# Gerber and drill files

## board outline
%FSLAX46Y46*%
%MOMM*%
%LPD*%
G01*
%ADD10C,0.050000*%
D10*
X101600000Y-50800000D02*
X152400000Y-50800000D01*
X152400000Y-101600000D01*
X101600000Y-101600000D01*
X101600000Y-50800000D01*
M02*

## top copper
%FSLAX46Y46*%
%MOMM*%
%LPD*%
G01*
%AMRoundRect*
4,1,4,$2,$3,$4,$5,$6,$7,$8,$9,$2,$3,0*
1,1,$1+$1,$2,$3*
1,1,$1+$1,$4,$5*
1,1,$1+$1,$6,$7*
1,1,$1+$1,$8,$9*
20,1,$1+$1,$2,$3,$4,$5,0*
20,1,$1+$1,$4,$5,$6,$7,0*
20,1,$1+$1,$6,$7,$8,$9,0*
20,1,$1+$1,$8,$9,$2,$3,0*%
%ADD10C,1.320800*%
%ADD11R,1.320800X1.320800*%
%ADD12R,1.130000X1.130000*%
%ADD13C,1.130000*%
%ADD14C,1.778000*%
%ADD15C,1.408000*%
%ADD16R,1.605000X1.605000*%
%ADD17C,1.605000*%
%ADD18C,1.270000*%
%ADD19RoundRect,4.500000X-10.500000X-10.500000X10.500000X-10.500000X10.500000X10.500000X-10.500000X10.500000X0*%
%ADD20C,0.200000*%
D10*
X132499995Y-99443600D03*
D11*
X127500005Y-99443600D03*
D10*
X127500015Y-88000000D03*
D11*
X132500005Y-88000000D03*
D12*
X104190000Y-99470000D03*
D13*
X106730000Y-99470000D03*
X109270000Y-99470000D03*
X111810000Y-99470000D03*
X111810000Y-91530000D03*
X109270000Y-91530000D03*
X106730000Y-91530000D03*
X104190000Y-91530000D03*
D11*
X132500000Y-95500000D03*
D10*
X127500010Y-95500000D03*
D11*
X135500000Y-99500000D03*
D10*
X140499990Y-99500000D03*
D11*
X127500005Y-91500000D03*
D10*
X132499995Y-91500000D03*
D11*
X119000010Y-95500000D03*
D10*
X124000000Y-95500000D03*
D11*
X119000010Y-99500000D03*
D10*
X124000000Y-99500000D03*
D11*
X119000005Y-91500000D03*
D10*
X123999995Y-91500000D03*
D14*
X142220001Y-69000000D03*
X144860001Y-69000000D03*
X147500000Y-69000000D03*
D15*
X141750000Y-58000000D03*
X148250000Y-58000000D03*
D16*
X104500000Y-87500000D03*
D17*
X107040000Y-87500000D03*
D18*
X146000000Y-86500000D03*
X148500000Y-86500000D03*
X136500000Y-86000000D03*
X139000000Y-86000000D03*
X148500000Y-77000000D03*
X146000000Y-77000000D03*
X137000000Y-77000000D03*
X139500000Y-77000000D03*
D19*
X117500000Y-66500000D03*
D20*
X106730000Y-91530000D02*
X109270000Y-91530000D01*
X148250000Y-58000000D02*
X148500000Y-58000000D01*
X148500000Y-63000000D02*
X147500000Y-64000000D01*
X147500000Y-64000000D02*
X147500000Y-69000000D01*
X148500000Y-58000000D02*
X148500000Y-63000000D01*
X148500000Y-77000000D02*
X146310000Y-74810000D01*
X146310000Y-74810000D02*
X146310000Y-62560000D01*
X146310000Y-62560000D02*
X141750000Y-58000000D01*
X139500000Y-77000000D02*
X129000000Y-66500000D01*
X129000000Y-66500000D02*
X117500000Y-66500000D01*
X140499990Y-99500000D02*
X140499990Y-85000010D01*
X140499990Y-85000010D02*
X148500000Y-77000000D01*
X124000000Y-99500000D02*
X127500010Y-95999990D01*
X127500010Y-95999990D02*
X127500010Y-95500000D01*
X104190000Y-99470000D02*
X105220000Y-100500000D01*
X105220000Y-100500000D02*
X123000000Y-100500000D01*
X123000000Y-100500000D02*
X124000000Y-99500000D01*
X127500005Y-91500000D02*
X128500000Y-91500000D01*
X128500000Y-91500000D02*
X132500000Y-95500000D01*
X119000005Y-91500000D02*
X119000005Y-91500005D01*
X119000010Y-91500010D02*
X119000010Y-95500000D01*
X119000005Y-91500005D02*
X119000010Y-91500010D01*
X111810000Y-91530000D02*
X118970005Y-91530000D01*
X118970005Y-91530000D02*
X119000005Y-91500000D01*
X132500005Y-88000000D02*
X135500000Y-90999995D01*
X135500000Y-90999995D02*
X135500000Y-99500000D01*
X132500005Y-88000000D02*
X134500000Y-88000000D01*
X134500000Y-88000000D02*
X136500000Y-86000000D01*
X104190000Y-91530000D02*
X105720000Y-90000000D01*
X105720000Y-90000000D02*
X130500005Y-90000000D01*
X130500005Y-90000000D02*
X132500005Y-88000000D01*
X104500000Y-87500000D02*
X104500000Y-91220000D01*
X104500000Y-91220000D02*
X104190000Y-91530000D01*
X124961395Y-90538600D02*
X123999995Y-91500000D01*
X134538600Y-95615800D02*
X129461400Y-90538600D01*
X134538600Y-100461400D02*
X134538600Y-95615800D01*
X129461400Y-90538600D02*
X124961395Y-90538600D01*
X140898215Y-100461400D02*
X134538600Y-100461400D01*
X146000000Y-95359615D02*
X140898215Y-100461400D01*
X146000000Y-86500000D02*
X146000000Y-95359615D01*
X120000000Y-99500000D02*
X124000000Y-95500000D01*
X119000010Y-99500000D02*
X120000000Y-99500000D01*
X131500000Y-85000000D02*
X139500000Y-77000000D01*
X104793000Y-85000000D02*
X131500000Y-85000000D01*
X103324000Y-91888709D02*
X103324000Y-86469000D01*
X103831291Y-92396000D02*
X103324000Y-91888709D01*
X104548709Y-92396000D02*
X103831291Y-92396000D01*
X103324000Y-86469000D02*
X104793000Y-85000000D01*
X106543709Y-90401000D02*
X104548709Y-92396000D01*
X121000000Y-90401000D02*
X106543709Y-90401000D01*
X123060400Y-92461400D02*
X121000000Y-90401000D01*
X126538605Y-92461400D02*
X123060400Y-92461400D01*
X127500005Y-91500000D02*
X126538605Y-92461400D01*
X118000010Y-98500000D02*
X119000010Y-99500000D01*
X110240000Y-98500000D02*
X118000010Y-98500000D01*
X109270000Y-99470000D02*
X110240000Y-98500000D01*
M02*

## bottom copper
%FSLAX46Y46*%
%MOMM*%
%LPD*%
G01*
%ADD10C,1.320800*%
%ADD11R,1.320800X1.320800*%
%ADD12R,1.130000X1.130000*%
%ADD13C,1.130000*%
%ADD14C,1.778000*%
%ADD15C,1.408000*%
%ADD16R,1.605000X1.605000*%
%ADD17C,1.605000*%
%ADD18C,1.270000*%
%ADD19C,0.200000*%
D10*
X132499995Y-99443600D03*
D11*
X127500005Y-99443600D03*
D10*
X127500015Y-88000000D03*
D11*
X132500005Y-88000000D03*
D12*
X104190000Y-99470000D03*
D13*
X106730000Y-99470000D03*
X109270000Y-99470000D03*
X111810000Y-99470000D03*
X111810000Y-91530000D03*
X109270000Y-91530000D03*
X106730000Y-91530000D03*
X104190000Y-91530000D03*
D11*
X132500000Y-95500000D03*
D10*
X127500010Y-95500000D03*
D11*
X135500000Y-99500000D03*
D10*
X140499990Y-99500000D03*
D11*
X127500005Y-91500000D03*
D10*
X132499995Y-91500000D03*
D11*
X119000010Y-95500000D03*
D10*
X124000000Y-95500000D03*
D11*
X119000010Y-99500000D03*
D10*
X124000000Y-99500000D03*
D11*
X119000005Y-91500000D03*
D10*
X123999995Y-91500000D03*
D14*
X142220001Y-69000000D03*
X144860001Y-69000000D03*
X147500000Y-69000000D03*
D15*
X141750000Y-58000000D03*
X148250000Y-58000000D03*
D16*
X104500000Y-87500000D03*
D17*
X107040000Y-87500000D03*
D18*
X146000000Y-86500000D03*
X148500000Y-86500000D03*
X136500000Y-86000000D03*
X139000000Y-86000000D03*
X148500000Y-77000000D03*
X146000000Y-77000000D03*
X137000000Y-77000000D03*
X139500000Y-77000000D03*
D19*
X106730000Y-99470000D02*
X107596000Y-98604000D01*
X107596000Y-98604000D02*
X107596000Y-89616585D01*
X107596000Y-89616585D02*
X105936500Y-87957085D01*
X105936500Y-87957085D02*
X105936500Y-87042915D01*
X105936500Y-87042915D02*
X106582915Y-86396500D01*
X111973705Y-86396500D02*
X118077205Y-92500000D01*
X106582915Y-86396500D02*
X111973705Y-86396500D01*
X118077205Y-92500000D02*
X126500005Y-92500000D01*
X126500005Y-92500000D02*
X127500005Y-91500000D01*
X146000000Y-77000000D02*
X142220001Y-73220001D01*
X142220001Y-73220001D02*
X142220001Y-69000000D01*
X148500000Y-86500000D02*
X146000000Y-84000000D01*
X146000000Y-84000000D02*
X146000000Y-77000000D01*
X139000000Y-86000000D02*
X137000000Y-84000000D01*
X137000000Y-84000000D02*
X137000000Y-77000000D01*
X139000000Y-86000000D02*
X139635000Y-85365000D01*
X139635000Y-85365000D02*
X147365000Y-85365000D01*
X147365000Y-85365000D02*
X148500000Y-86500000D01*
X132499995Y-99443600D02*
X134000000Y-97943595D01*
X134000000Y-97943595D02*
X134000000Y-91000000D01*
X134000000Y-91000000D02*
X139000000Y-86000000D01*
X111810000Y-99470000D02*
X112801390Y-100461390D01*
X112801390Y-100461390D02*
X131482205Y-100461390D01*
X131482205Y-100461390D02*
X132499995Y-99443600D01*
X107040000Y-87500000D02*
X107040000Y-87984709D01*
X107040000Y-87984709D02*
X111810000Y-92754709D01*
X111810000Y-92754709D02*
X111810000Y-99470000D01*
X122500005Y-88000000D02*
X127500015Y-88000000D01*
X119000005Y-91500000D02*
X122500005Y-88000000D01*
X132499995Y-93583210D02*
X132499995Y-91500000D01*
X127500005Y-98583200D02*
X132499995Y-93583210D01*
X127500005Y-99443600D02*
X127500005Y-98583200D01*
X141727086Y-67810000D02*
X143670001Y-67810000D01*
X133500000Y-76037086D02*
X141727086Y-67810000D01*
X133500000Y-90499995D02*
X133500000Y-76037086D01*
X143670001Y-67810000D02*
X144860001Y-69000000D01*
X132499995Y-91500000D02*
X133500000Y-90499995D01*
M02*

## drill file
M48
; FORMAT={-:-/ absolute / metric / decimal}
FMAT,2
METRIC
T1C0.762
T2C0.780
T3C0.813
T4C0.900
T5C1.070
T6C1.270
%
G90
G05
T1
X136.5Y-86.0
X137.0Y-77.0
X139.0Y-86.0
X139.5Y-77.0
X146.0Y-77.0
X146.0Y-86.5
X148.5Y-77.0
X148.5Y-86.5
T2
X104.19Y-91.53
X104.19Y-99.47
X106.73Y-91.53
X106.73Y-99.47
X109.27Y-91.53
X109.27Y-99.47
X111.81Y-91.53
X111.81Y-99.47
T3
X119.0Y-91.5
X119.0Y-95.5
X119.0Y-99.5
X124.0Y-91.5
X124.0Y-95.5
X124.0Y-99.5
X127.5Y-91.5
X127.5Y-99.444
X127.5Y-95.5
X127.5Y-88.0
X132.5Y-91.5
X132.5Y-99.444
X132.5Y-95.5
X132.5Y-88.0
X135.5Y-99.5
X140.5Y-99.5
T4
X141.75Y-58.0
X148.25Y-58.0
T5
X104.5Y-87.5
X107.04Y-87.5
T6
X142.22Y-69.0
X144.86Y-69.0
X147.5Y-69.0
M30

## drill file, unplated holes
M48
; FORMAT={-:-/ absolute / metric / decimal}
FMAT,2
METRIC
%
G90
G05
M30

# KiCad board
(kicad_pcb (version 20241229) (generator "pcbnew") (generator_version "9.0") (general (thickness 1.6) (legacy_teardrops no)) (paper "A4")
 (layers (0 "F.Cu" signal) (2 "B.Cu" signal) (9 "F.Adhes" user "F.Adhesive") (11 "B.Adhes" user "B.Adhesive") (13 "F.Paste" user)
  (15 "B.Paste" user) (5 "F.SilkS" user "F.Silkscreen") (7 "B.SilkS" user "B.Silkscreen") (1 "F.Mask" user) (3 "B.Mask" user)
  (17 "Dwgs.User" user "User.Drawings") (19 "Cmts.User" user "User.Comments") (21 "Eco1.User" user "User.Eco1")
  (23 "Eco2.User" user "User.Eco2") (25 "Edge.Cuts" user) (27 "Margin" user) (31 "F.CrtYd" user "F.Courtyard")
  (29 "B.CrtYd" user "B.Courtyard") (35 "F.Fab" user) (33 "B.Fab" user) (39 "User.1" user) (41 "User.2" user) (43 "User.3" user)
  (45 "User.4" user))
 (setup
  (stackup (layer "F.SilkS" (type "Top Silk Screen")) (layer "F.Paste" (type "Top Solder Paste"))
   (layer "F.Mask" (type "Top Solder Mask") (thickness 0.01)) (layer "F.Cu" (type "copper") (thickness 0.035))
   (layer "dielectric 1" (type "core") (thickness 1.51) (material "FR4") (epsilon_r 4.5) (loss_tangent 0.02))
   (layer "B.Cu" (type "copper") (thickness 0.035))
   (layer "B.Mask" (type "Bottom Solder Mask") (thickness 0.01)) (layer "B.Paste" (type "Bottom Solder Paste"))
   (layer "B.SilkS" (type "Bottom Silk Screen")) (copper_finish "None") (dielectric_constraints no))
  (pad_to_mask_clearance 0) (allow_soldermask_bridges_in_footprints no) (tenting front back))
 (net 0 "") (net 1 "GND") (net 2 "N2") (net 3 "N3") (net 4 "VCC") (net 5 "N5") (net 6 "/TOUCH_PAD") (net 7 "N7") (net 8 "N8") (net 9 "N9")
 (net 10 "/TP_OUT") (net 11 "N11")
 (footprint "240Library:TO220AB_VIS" (layer "F.Cu") (at 142.220001 69)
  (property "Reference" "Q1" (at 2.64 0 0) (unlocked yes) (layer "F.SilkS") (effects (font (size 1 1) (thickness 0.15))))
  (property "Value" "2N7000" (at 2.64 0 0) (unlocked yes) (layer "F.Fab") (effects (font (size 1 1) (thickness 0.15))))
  (pad "1" thru_hole circle (at 0 0) (size 1.778 1.778) (drill 1.27) (layers "*.Cu" "*.Mask") (remove_unused_layers no) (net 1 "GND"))
  (pad "2" thru_hole circle (at 2.64 0) (size 1.778 1.778) (drill 1.27) (layers "*.Cu" "*.Mask") (remove_unused_layers no) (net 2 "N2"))
  (pad "3" thru_hole circle (at 5.279999 0) (size 1.778 1.778) (drill 1.27) (layers "*.Cu" "*.Mask") (remove_unused_layers no) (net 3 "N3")))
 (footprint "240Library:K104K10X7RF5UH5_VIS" (layer "F.Cu") (at 132.500005 88 180)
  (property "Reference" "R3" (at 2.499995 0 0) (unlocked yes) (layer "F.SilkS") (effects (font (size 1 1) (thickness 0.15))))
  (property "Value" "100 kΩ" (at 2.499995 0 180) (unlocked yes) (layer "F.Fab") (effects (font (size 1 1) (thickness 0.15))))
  (pad "1" thru_hole rect (at 0 0 180) (size 1.3208 1.3208) (drill 0.8128) (layers "*.Cu" "*.Mask") (remove_unused_layers no) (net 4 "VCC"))
  (pad "2" thru_hole circle (at 4.99999 0 180) (size 1.3208 1.3208) (drill 0.8128) (layers "*.Cu" "*.Mask") (remove_unused_layers no)
   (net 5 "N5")))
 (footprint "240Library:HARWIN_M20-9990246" (layer "F.Cu") (at 105.77 87.5)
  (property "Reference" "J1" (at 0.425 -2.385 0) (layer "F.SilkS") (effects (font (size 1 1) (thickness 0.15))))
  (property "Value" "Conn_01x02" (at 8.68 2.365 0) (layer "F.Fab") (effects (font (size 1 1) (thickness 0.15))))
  (pad "1" thru_hole rect (at -1.27 0) (size 1.605 1.605) (drill 1.07) (layers "*.Cu" "*.Mask") (remove_unused_layers no) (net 4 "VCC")
   (solder_mask_margin 0.102))
  (pad "2" thru_hole circle (at 1.27 0) (size 1.605 1.605) (drill 1.07) (layers "*.Cu" "*.Mask") (remove_unused_layers no) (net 1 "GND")
   (solder_mask_margin 0.102)))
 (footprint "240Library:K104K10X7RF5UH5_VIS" (layer "F.Cu") (at 127.500005 91.5)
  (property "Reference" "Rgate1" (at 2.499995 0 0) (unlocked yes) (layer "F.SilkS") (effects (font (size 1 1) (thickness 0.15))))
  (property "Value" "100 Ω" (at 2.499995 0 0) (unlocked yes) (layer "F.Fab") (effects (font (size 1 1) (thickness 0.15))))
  (pad "1" thru_hole rect (at 0 0) (size 1.3208 1.3208) (drill 0.8128) (layers "*.Cu" "*.Mask") (remove_unused_layers no)
   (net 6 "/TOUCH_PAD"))
  (pad "2" thru_hole circle (at 4.99999 0) (size 1.3208 1.3208) (drill 0.8128) (layers "*.Cu" "*.Mask") (remove_unused_layers no)
   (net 2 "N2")))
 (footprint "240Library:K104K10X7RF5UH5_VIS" (layer "F.Cu") (at 135.5 99.5)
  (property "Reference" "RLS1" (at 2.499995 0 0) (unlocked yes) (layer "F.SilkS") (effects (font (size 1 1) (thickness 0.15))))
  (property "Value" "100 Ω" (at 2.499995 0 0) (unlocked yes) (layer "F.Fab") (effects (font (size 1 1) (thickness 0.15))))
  (pad "1" thru_hole rect (at 0 0) (size 1.3208 1.3208) (drill 0.8128) (layers "*.Cu" "*.Mask") (remove_unused_layers no) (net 4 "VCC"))
  (pad "2" thru_hole circle (at 4.99999 0) (size 1.3208 1.3208) (drill 0.8128) (layers "*.Cu" "*.Mask") (remove_unused_layers no)
   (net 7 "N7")))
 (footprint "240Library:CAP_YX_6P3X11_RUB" (layer "F.Cu") (at 148.5 77 180)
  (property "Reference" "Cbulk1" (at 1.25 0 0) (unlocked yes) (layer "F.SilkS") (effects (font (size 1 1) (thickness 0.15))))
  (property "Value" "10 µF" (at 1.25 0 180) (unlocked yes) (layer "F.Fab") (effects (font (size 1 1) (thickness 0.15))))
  (pad "1" thru_hole circle (at 0 0 180) (size 1.27 1.27) (drill 0.762) (layers "*.Cu" "*.Mask") (remove_unused_layers no) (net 7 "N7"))
  (pad "2" thru_hole circle (at 2.5 0 180) (size 1.27 1.27) (drill 0.762) (layers "*.Cu" "*.Mask") (remove_unused_layers no) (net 1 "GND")))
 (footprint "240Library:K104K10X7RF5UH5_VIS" (layer "F.Cu") (at 119.00001 95.5)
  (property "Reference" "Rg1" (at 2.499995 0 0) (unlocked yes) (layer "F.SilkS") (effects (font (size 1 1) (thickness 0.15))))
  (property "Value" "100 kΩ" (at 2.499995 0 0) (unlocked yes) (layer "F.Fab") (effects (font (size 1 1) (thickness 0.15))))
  (pad "1" thru_hole rect (at 0 0) (size 1.3208 1.3208) (drill 0.8128) (layers "*.Cu" "*.Mask") (remove_unused_layers no) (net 5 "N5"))
  (pad "2" thru_hole circle (at 4.99999 0) (size 1.3208 1.3208) (drill 0.8128) (layers "*.Cu" "*.Mask") (remove_unused_layers no)
   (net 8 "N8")))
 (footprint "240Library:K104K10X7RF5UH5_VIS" (layer "F.Cu") (at 119.000005 91.5)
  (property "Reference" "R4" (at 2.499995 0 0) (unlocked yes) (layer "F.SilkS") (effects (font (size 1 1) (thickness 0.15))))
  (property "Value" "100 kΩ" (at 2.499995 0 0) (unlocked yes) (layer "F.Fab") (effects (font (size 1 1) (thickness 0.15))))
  (pad "1" thru_hole rect (at 0 0) (size 1.3208 1.3208) (drill 0.8128) (layers "*.Cu" "*.Mask") (remove_unused_layers no) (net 5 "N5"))
  (pad "2" thru_hole circle (at 4.99999 0) (size 1.3208 1.3208) (drill 0.8128) (layers "*.Cu" "*.Mask") (remove_unused_layers no)
   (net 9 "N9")))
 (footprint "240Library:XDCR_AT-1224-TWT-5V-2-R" (layer "F.Cu") (at 145 58 90)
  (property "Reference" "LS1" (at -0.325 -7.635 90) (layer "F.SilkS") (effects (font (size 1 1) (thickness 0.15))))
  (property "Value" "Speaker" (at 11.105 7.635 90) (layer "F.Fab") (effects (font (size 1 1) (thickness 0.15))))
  (pad "1" thru_hole circle (at 0 -3.25 90) (size 1.408 1.408) (drill 0.9) (layers "*.Cu" "*.Mask") (remove_unused_layers no) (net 7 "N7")
   (solder_mask_margin 0.102))
  (pad "2" thru_hole circle (at 0 3.25 90) (size 1.408 1.408) (drill 0.9) (layers "*.Cu" "*.Mask") (remove_unused_layers no) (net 3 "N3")
   (solder_mask_margin 0.102)))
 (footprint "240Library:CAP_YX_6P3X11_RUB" (layer "F.Cu") (at 136.5 86)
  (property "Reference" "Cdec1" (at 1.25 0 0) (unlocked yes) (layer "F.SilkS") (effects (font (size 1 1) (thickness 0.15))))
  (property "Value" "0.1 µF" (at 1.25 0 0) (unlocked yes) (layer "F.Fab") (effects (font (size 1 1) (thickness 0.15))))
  (pad "1" thru_hole circle (at 0 0) (size 1.27 1.27) (drill 0.762) (layers "*.Cu" "*.Mask") (remove_unused_layers no) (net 4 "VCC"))
  (pad "2" thru_hole circle (at 2.5 0) (size 1.27 1.27) (drill 0.762) (layers "*.Cu" "*.Mask") (remove_unused_layers no) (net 1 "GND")))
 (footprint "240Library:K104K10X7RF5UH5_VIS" (layer "F.Cu") (at 132.5 95.5 180)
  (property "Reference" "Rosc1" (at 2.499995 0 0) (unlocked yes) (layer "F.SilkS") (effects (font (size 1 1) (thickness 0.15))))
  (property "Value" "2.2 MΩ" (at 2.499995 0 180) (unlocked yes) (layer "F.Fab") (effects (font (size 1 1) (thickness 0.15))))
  (pad "1" thru_hole rect (at 0 0 180) (size 1.3208 1.3208) (drill 0.8128) (layers "*.Cu" "*.Mask") (remove_unused_layers no)
   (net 6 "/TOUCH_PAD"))
  (pad "2" thru_hole circle (at 4.99999 0 180) (size 1.3208 1.3208) (drill 0.8128) (layers "*.Cu" "*.Mask") (remove_unused_layers no)
   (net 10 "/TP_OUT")))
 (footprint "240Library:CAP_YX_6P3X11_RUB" (layer "F.Cu") (at 146 86.5)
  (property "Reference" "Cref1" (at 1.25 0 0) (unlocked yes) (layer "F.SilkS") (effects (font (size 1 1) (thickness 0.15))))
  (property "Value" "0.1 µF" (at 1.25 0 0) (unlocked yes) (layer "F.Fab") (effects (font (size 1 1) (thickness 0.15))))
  (pad "1" thru_hole circle (at 0 0) (size 1.27 1.27) (drill 0.762) (layers "*.Cu" "*.Mask") (remove_unused_layers no) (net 9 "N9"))
  (pad "2" thru_hole circle (at 2.5 0) (size 1.27 1.27) (drill 0.762) (layers "*.Cu" "*.Mask") (remove_unused_layers no) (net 1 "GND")))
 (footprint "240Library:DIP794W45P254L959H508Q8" (layer "F.Cu") (at 108 95.5 90)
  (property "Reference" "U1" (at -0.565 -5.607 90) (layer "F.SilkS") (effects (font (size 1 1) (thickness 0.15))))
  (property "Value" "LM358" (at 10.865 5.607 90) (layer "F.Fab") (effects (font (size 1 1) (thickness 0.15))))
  (pad "1" thru_hole rect (at -3.97 -3.81 90) (size 1.13 1.13) (drill 0.78) (layers "*.Cu" "*.Mask") (remove_unused_layers no)
   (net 10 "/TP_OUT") (solder_mask_margin 0.102))
  (pad "2" thru_hole circle (at -3.97 -1.27 90) (size 1.13 1.13) (drill 0.78) (layers "*.Cu" "*.Mask") (remove_unused_layers no)
   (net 6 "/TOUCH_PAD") (solder_mask_margin 0.102))
  (pad "3" thru_hole circle (at -3.97 1.27 90) (size 1.13 1.13) (drill 0.78) (layers "*.Cu" "*.Mask") (remove_unused_layers no) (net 8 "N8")
   (solder_mask_margin 0.102))
  (pad "4" thru_hole circle (at -3.97 3.81 90) (size 1.13 1.13) (drill 0.78) (layers "*.Cu" "*.Mask") (remove_unused_layers no)
   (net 1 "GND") (solder_mask_margin 0.102))
  (pad "5" thru_hole circle (at 3.97 3.81 90) (size 1.13 1.13) (drill 0.78) (layers "*.Cu" "*.Mask") (remove_unused_layers no) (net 5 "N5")
   (solder_mask_margin 0.102))
  (pad "6" thru_hole circle (at 3.97 1.27 90) (size 1.13 1.13) (drill 0.78) (layers "*.Cu" "*.Mask") (remove_unused_layers no)
   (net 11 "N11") (solder_mask_margin 0.102))
  (pad "7" thru_hole circle (at 3.97 -1.27 90) (size 1.13 1.13) (drill 0.78) (layers "*.Cu" "*.Mask") (remove_unused_layers no)
   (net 11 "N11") (solder_mask_margin 0.102))
  (pad "8" thru_hole circle (at 3.97 -3.81 90) (size 1.13 1.13) (drill 0.78) (layers "*.Cu" "*.Mask") (remove_unused_layers no)
   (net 4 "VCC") (solder_mask_margin 0.102)))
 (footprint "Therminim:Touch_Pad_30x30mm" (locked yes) (layer "F.Cu") (at 117.5 66.5)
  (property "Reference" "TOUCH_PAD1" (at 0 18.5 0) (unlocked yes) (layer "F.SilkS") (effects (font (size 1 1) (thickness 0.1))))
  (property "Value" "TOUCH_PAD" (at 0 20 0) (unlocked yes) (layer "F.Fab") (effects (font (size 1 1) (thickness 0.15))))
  (pad "1" smd roundrect (at 0 0) (size 30 30) (layers "F.Cu" "F.Mask") (roundrect_rratio 0.15) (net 6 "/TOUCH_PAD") (clearance 1)))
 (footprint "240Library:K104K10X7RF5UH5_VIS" (layer "F.Cu") (at 119.00001 99.5)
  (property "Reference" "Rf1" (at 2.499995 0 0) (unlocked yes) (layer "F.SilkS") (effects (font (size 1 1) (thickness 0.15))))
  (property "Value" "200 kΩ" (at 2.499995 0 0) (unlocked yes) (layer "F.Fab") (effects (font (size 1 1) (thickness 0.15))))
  (pad "1" thru_hole rect (at 0 0) (size 1.3208 1.3208) (drill 0.8128) (layers "*.Cu" "*.Mask") (remove_unused_layers no) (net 8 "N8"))
  (pad "2" thru_hole circle (at 4.99999 0) (size 1.3208 1.3208) (drill 0.8128) (layers "*.Cu" "*.Mask") (remove_unused_layers no)
   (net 10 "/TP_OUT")))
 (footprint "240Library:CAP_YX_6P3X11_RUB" (layer "F.Cu") (at 137 77)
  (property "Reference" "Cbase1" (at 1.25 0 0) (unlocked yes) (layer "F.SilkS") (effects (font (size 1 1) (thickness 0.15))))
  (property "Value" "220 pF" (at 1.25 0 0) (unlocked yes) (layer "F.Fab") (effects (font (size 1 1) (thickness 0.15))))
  (pad "1" thru_hole circle (at 0 0) (size 1.27 1.27) (drill 0.762) (layers "*.Cu" "*.Mask") (remove_unused_layers no) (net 1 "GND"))
  (pad "2" thru_hole circle (at 2.5 0) (size 1.27 1.27) (drill 0.762) (layers "*.Cu" "*.Mask") (remove_unused_layers no)
   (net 6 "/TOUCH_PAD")))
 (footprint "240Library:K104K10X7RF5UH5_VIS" (layer "F.Cu") (at 127.500005 99.4436)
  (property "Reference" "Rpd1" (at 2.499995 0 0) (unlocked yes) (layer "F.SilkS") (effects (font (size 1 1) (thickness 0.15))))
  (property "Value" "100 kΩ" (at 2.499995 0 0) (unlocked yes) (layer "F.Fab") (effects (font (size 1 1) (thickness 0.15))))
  (pad "1" thru_hole rect (at 0 0) (size 1.3208 1.3208) (drill 0.8128) (layers "*.Cu" "*.Mask") (remove_unused_layers no) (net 2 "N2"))
  (pad "2" thru_hole circle (at 4.99999 0) (size 1.3208 1.3208) (drill 0.8128) (layers "*.Cu" "*.Mask") (remove_unused_layers no)
   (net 1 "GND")))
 (gr_rect (start 101.6 50.8) (end 152.4 101.6) (stroke (width 0.05) (type solid)) (fill no) (layer "Edge.Cuts"))
 (segment (start 142.220001 73.220001) (end 142.220001 69) (width 0.2) (layer "B.Cu") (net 1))
 (segment (start 148.5 86.5) (end 146 84) (width 0.2) (layer "B.Cu") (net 1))
 (segment (start 139 86) (end 137 84) (width 0.2) (layer "B.Cu") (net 1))
 (segment (start 112.80139 100.46139) (end 131.482205 100.46139) (width 0.2) (layer "B.Cu") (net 1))
 (segment (start 132.499995 99.4436) (end 134 97.943595) (width 0.2) (layer "B.Cu") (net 1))
 (segment (start 134 97.943595) (end 134 91) (width 0.2) (layer "B.Cu") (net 1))
 (segment (start 146 84) (end 146 77) (width 0.2) (layer "B.Cu") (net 1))
 (segment (start 111.81 92.754709) (end 111.81 99.47) (width 0.2) (layer "B.Cu") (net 1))
 (segment (start 111.81 99.47) (end 112.80139 100.46139) (width 0.2) (layer "B.Cu") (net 1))
 (segment (start 131.482205 100.46139) (end 132.499995 99.4436) (width 0.2) (layer "B.Cu") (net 1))
 (segment (start 134 91) (end 139 86) (width 0.2) (layer "B.Cu") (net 1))
 (segment (start 146 77) (end 142.220001 73.220001) (width 0.2) (layer "B.Cu") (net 1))
 (segment (start 147.365 85.365) (end 148.5 86.5) (width 0.2) (layer "B.Cu") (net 1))
 (segment (start 107.04 87.984709) (end 111.81 92.754709) (width 0.2) (layer "B.Cu") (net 1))
 (segment (start 107.04 87.5) (end 107.04 87.984709) (width 0.2) (layer "B.Cu") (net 1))
 (segment (start 137 84) (end 137 77) (width 0.2) (layer "B.Cu") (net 1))
 (segment (start 139 86) (end 139.635 85.365) (width 0.2) (layer "B.Cu") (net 1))
 (segment (start 139.635 85.365) (end 147.365 85.365) (width 0.2) (layer "B.Cu") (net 1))
 (segment (start 104.548709 92.396) (end 103.831291 92.396) (width 0.2) (layer "F.Cu") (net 6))
 (segment (start 126.538605 92.4614) (end 123.0604 92.4614) (width 0.2) (layer "F.Cu") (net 6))
 (segment (start 103.324 86.469) (end 104.793 85) (width 0.2) (layer "F.Cu") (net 6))
 (segment (start 103.324 91.888709) (end 103.324 86.469) (width 0.2) (layer "F.Cu") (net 6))
 (segment (start 121 90.401) (end 106.543709 90.401) (width 0.2) (layer "F.Cu") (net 6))
 (segment (start 106.543709 90.401) (end 104.548709 92.396) (width 0.2) (layer "F.Cu") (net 6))
 (segment (start 123.0604 92.4614) (end 121 90.401) (width 0.2) (layer "F.Cu") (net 6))
 (segment (start 127.500005 91.5) (end 128.5 91.5) (width 0.2) (layer "F.Cu") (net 6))
 (segment (start 103.831291 92.396) (end 103.324 91.888709) (width 0.2) (layer "F.Cu") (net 6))
 (segment (start 131.5 85) (end 139.5 77) (width 0.2) (layer "F.Cu") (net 6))
 (segment (start 127.500005 91.5) (end 126.538605 92.4614) (width 0.2) (layer "F.Cu") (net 6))
 (segment (start 129 66.5) (end 117.5 66.5) (width 0.2) (layer "F.Cu") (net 6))
 (segment (start 139.5 77) (end 129 66.5) (width 0.2) (layer "F.Cu") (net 6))
 (segment (start 128.5 91.5) (end 132.5 95.5) (width 0.2) (layer "F.Cu") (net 6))
 (segment (start 104.793 85) (end 131.5 85) (width 0.2) (layer "F.Cu") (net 6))
 (segment (start 107.596 89.616585) (end 105.9365 87.957085) (width 0.2) (layer "B.Cu") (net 6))
 (segment (start 106.73 99.47) (end 107.596 98.604) (width 0.2) (layer "B.Cu") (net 6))
 (segment (start 105.9365 87.957085) (end 105.9365 87.042915) (width 0.2) (layer "B.Cu") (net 6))
 (segment (start 118.077205 92.5) (end 126.500005 92.5) (width 0.2) (layer "B.Cu") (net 6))
 (segment (start 126.500005 92.5) (end 127.500005 91.5) (width 0.2) (layer "B.Cu") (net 6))
 (segment (start 107.596 98.604) (end 107.596 89.616585) (width 0.2) (layer "B.Cu") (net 6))
 (segment (start 105.9365 87.042915) (end 106.582915 86.3965) (width 0.2) (layer "B.Cu") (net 6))
 (segment (start 106.582915 86.3965) (end 111.973705 86.3965) (width 0.2) (layer "B.Cu") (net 6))
 (segment (start 111.973705 86.3965) (end 118.077205 92.5) (width 0.2) (layer "B.Cu") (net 6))
 (segment (start 148.5 77) (end 146.31 74.81) (width 0.2) (layer "F.Cu") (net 7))
 (segment (start 146.31 74.81) (end 146.31 62.56) (width 0.2) (layer "F.Cu") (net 7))
 (segment (start 140.49999 99.5) (end 140.49999 85.00001) (width 0.2) (layer "F.Cu") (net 7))
 (segment (start 146.31 62.56) (end 141.75 58) (width 0.2) (layer "F.Cu") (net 7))
 (segment (start 140.49999 85.00001) (end 148.5 77) (width 0.2) (layer "F.Cu") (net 7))
 (segment (start 132.500005 88) (end 134.5 88) (width 0.2) (layer "F.Cu") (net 4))
 (segment (start 134.5 88) (end 136.5 86) (width 0.2) (layer "F.Cu") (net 4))
 (segment (start 135.5 90.999995) (end 135.5 99.5) (width 0.2) (layer "F.Cu") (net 4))
 (segment (start 104.5 87.5) (end 104.5 91.22) (width 0.2) (layer "F.Cu") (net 4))
 (segment (start 104.5 91.22) (end 104.19 91.53) (width 0.2) (layer "F.Cu") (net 4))
 (segment (start 104.19 91.53) (end 105.72 90) (width 0.2) (layer "F.Cu") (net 4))
 (segment (start 132.500005 88) (end 135.5 90.999995) (width 0.2) (layer "F.Cu") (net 4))
 (segment (start 130.500005 90) (end 132.500005 88) (width 0.2) (layer "F.Cu") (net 4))
 (segment (start 105.72 90) (end 130.500005 90) (width 0.2) (layer "F.Cu") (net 4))
 (segment (start 146 86.5) (end 146 95.359615) (width 0.2) (layer "F.Cu") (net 9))
 (segment (start 129.4614 90.5386) (end 124.961395 90.5386) (width 0.2) (layer "F.Cu") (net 9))
 (segment (start 146 95.359615) (end 140.898215 100.4614) (width 0.2) (layer "F.Cu") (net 9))
 (segment (start 134.5386 95.6158) (end 129.4614 90.5386) (width 0.2) (layer "F.Cu") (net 9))
 (segment (start 140.898215 100.4614) (end 134.5386 100.4614) (width 0.2) (layer "F.Cu") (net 9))
 (segment (start 124.961395 90.5386) (end 123.999995 91.5) (width 0.2) (layer "F.Cu") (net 9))
 (segment (start 134.5386 100.4614) (end 134.5386 95.6158) (width 0.2) (layer "F.Cu") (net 9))
 (segment (start 148.5 58) (end 148.5 63) (width 0.2) (layer "F.Cu") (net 3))
 (segment (start 148.5 63) (end 147.5 64) (width 0.2) (layer "F.Cu") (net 3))
 (segment (start 147.5 64) (end 147.5 69) (width 0.2) (layer "F.Cu") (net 3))
 (segment (start 148.25 58) (end 148.5 58) (width 0.2) (layer "F.Cu") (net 3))
 (segment (start 127.500005 98.5832) (end 132.499995 93.58321) (width 0.2) (layer "B.Cu") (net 2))
 (segment (start 132.499995 93.58321) (end 132.499995 91.5) (width 0.2) (layer "B.Cu") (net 2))
 (segment (start 141.727086 67.81) (end 143.670001 67.81) (width 0.2) (layer "B.Cu") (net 2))
 (segment (start 132.499995 91.5) (end 133.5 90.499995) (width 0.2) (layer "B.Cu") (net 2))
 (segment (start 133.5 90.499995) (end 133.5 76.037086) (width 0.2) (layer "B.Cu") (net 2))
 (segment (start 143.670001 67.81) (end 144.860001 69) (width 0.2) (layer "B.Cu") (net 2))
 (segment (start 133.5 76.037086) (end 141.727086 67.81) (width 0.2) (layer "B.Cu") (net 2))
 (segment (start 127.500005 99.4436) (end 127.500005 98.5832) (width 0.2) (layer "B.Cu") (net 2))
 (segment (start 119.000005 91.5) (end 119.000005 91.500005) (width 0.2) (layer "F.Cu") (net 5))
 (segment (start 111.81 91.53) (end 118.970005 91.53) (width 0.2) (layer "F.Cu") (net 5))
 (segment (start 118.970005 91.53) (end 119.000005 91.5) (width 0.2) (layer "F.Cu") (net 5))
 (segment (start 119.00001 91.50001) (end 119.00001 95.5) (width 0.2) (layer "F.Cu") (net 5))
 (segment (start 119.000005 91.500005) (end 119.00001 91.50001) (width 0.2) (layer "F.Cu") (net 5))
 (segment (start 119.000005 91.5) (end 122.500005 88) (width 0.2) (layer "B.Cu") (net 5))
 (segment (start 122.500005 88) (end 127.500015 88) (width 0.2) (layer "B.Cu") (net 5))
 (segment (start 119.00001 99.5) (end 120 99.5) (width 0.2) (layer "F.Cu") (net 8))
 (segment (start 109.27 99.47) (end 110.24 98.5) (width 0.2) (layer "F.Cu") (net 8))
 (segment (start 110.24 98.5) (end 118.00001 98.5) (width 0.2) (layer "F.Cu") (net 8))
 (segment (start 118.00001 98.5) (end 119.00001 99.5) (width 0.2) (layer "F.Cu") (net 8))
 (segment (start 120 99.5) (end 124 95.5) (width 0.2) (layer "F.Cu") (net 8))
 (segment (start 127.50001 95.99999) (end 127.50001 95.5) (width 0.2) (layer "F.Cu") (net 10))
 (segment (start 105.22 100.5) (end 123 100.5) (width 0.2) (layer "F.Cu") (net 10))
 (segment (start 104.19 99.47) (end 105.22 100.5) (width 0.2) (layer "F.Cu") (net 10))
 (segment (start 124 99.5) (end 127.50001 95.99999) (width 0.2) (layer "F.Cu") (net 10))
 (segment (start 123 100.5) (end 124 99.5) (width 0.2) (layer "F.Cu") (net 10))
 (segment (start 106.73 91.53) (end 109.27 91.53) (width 0.2) (layer "F.Cu") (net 11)))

